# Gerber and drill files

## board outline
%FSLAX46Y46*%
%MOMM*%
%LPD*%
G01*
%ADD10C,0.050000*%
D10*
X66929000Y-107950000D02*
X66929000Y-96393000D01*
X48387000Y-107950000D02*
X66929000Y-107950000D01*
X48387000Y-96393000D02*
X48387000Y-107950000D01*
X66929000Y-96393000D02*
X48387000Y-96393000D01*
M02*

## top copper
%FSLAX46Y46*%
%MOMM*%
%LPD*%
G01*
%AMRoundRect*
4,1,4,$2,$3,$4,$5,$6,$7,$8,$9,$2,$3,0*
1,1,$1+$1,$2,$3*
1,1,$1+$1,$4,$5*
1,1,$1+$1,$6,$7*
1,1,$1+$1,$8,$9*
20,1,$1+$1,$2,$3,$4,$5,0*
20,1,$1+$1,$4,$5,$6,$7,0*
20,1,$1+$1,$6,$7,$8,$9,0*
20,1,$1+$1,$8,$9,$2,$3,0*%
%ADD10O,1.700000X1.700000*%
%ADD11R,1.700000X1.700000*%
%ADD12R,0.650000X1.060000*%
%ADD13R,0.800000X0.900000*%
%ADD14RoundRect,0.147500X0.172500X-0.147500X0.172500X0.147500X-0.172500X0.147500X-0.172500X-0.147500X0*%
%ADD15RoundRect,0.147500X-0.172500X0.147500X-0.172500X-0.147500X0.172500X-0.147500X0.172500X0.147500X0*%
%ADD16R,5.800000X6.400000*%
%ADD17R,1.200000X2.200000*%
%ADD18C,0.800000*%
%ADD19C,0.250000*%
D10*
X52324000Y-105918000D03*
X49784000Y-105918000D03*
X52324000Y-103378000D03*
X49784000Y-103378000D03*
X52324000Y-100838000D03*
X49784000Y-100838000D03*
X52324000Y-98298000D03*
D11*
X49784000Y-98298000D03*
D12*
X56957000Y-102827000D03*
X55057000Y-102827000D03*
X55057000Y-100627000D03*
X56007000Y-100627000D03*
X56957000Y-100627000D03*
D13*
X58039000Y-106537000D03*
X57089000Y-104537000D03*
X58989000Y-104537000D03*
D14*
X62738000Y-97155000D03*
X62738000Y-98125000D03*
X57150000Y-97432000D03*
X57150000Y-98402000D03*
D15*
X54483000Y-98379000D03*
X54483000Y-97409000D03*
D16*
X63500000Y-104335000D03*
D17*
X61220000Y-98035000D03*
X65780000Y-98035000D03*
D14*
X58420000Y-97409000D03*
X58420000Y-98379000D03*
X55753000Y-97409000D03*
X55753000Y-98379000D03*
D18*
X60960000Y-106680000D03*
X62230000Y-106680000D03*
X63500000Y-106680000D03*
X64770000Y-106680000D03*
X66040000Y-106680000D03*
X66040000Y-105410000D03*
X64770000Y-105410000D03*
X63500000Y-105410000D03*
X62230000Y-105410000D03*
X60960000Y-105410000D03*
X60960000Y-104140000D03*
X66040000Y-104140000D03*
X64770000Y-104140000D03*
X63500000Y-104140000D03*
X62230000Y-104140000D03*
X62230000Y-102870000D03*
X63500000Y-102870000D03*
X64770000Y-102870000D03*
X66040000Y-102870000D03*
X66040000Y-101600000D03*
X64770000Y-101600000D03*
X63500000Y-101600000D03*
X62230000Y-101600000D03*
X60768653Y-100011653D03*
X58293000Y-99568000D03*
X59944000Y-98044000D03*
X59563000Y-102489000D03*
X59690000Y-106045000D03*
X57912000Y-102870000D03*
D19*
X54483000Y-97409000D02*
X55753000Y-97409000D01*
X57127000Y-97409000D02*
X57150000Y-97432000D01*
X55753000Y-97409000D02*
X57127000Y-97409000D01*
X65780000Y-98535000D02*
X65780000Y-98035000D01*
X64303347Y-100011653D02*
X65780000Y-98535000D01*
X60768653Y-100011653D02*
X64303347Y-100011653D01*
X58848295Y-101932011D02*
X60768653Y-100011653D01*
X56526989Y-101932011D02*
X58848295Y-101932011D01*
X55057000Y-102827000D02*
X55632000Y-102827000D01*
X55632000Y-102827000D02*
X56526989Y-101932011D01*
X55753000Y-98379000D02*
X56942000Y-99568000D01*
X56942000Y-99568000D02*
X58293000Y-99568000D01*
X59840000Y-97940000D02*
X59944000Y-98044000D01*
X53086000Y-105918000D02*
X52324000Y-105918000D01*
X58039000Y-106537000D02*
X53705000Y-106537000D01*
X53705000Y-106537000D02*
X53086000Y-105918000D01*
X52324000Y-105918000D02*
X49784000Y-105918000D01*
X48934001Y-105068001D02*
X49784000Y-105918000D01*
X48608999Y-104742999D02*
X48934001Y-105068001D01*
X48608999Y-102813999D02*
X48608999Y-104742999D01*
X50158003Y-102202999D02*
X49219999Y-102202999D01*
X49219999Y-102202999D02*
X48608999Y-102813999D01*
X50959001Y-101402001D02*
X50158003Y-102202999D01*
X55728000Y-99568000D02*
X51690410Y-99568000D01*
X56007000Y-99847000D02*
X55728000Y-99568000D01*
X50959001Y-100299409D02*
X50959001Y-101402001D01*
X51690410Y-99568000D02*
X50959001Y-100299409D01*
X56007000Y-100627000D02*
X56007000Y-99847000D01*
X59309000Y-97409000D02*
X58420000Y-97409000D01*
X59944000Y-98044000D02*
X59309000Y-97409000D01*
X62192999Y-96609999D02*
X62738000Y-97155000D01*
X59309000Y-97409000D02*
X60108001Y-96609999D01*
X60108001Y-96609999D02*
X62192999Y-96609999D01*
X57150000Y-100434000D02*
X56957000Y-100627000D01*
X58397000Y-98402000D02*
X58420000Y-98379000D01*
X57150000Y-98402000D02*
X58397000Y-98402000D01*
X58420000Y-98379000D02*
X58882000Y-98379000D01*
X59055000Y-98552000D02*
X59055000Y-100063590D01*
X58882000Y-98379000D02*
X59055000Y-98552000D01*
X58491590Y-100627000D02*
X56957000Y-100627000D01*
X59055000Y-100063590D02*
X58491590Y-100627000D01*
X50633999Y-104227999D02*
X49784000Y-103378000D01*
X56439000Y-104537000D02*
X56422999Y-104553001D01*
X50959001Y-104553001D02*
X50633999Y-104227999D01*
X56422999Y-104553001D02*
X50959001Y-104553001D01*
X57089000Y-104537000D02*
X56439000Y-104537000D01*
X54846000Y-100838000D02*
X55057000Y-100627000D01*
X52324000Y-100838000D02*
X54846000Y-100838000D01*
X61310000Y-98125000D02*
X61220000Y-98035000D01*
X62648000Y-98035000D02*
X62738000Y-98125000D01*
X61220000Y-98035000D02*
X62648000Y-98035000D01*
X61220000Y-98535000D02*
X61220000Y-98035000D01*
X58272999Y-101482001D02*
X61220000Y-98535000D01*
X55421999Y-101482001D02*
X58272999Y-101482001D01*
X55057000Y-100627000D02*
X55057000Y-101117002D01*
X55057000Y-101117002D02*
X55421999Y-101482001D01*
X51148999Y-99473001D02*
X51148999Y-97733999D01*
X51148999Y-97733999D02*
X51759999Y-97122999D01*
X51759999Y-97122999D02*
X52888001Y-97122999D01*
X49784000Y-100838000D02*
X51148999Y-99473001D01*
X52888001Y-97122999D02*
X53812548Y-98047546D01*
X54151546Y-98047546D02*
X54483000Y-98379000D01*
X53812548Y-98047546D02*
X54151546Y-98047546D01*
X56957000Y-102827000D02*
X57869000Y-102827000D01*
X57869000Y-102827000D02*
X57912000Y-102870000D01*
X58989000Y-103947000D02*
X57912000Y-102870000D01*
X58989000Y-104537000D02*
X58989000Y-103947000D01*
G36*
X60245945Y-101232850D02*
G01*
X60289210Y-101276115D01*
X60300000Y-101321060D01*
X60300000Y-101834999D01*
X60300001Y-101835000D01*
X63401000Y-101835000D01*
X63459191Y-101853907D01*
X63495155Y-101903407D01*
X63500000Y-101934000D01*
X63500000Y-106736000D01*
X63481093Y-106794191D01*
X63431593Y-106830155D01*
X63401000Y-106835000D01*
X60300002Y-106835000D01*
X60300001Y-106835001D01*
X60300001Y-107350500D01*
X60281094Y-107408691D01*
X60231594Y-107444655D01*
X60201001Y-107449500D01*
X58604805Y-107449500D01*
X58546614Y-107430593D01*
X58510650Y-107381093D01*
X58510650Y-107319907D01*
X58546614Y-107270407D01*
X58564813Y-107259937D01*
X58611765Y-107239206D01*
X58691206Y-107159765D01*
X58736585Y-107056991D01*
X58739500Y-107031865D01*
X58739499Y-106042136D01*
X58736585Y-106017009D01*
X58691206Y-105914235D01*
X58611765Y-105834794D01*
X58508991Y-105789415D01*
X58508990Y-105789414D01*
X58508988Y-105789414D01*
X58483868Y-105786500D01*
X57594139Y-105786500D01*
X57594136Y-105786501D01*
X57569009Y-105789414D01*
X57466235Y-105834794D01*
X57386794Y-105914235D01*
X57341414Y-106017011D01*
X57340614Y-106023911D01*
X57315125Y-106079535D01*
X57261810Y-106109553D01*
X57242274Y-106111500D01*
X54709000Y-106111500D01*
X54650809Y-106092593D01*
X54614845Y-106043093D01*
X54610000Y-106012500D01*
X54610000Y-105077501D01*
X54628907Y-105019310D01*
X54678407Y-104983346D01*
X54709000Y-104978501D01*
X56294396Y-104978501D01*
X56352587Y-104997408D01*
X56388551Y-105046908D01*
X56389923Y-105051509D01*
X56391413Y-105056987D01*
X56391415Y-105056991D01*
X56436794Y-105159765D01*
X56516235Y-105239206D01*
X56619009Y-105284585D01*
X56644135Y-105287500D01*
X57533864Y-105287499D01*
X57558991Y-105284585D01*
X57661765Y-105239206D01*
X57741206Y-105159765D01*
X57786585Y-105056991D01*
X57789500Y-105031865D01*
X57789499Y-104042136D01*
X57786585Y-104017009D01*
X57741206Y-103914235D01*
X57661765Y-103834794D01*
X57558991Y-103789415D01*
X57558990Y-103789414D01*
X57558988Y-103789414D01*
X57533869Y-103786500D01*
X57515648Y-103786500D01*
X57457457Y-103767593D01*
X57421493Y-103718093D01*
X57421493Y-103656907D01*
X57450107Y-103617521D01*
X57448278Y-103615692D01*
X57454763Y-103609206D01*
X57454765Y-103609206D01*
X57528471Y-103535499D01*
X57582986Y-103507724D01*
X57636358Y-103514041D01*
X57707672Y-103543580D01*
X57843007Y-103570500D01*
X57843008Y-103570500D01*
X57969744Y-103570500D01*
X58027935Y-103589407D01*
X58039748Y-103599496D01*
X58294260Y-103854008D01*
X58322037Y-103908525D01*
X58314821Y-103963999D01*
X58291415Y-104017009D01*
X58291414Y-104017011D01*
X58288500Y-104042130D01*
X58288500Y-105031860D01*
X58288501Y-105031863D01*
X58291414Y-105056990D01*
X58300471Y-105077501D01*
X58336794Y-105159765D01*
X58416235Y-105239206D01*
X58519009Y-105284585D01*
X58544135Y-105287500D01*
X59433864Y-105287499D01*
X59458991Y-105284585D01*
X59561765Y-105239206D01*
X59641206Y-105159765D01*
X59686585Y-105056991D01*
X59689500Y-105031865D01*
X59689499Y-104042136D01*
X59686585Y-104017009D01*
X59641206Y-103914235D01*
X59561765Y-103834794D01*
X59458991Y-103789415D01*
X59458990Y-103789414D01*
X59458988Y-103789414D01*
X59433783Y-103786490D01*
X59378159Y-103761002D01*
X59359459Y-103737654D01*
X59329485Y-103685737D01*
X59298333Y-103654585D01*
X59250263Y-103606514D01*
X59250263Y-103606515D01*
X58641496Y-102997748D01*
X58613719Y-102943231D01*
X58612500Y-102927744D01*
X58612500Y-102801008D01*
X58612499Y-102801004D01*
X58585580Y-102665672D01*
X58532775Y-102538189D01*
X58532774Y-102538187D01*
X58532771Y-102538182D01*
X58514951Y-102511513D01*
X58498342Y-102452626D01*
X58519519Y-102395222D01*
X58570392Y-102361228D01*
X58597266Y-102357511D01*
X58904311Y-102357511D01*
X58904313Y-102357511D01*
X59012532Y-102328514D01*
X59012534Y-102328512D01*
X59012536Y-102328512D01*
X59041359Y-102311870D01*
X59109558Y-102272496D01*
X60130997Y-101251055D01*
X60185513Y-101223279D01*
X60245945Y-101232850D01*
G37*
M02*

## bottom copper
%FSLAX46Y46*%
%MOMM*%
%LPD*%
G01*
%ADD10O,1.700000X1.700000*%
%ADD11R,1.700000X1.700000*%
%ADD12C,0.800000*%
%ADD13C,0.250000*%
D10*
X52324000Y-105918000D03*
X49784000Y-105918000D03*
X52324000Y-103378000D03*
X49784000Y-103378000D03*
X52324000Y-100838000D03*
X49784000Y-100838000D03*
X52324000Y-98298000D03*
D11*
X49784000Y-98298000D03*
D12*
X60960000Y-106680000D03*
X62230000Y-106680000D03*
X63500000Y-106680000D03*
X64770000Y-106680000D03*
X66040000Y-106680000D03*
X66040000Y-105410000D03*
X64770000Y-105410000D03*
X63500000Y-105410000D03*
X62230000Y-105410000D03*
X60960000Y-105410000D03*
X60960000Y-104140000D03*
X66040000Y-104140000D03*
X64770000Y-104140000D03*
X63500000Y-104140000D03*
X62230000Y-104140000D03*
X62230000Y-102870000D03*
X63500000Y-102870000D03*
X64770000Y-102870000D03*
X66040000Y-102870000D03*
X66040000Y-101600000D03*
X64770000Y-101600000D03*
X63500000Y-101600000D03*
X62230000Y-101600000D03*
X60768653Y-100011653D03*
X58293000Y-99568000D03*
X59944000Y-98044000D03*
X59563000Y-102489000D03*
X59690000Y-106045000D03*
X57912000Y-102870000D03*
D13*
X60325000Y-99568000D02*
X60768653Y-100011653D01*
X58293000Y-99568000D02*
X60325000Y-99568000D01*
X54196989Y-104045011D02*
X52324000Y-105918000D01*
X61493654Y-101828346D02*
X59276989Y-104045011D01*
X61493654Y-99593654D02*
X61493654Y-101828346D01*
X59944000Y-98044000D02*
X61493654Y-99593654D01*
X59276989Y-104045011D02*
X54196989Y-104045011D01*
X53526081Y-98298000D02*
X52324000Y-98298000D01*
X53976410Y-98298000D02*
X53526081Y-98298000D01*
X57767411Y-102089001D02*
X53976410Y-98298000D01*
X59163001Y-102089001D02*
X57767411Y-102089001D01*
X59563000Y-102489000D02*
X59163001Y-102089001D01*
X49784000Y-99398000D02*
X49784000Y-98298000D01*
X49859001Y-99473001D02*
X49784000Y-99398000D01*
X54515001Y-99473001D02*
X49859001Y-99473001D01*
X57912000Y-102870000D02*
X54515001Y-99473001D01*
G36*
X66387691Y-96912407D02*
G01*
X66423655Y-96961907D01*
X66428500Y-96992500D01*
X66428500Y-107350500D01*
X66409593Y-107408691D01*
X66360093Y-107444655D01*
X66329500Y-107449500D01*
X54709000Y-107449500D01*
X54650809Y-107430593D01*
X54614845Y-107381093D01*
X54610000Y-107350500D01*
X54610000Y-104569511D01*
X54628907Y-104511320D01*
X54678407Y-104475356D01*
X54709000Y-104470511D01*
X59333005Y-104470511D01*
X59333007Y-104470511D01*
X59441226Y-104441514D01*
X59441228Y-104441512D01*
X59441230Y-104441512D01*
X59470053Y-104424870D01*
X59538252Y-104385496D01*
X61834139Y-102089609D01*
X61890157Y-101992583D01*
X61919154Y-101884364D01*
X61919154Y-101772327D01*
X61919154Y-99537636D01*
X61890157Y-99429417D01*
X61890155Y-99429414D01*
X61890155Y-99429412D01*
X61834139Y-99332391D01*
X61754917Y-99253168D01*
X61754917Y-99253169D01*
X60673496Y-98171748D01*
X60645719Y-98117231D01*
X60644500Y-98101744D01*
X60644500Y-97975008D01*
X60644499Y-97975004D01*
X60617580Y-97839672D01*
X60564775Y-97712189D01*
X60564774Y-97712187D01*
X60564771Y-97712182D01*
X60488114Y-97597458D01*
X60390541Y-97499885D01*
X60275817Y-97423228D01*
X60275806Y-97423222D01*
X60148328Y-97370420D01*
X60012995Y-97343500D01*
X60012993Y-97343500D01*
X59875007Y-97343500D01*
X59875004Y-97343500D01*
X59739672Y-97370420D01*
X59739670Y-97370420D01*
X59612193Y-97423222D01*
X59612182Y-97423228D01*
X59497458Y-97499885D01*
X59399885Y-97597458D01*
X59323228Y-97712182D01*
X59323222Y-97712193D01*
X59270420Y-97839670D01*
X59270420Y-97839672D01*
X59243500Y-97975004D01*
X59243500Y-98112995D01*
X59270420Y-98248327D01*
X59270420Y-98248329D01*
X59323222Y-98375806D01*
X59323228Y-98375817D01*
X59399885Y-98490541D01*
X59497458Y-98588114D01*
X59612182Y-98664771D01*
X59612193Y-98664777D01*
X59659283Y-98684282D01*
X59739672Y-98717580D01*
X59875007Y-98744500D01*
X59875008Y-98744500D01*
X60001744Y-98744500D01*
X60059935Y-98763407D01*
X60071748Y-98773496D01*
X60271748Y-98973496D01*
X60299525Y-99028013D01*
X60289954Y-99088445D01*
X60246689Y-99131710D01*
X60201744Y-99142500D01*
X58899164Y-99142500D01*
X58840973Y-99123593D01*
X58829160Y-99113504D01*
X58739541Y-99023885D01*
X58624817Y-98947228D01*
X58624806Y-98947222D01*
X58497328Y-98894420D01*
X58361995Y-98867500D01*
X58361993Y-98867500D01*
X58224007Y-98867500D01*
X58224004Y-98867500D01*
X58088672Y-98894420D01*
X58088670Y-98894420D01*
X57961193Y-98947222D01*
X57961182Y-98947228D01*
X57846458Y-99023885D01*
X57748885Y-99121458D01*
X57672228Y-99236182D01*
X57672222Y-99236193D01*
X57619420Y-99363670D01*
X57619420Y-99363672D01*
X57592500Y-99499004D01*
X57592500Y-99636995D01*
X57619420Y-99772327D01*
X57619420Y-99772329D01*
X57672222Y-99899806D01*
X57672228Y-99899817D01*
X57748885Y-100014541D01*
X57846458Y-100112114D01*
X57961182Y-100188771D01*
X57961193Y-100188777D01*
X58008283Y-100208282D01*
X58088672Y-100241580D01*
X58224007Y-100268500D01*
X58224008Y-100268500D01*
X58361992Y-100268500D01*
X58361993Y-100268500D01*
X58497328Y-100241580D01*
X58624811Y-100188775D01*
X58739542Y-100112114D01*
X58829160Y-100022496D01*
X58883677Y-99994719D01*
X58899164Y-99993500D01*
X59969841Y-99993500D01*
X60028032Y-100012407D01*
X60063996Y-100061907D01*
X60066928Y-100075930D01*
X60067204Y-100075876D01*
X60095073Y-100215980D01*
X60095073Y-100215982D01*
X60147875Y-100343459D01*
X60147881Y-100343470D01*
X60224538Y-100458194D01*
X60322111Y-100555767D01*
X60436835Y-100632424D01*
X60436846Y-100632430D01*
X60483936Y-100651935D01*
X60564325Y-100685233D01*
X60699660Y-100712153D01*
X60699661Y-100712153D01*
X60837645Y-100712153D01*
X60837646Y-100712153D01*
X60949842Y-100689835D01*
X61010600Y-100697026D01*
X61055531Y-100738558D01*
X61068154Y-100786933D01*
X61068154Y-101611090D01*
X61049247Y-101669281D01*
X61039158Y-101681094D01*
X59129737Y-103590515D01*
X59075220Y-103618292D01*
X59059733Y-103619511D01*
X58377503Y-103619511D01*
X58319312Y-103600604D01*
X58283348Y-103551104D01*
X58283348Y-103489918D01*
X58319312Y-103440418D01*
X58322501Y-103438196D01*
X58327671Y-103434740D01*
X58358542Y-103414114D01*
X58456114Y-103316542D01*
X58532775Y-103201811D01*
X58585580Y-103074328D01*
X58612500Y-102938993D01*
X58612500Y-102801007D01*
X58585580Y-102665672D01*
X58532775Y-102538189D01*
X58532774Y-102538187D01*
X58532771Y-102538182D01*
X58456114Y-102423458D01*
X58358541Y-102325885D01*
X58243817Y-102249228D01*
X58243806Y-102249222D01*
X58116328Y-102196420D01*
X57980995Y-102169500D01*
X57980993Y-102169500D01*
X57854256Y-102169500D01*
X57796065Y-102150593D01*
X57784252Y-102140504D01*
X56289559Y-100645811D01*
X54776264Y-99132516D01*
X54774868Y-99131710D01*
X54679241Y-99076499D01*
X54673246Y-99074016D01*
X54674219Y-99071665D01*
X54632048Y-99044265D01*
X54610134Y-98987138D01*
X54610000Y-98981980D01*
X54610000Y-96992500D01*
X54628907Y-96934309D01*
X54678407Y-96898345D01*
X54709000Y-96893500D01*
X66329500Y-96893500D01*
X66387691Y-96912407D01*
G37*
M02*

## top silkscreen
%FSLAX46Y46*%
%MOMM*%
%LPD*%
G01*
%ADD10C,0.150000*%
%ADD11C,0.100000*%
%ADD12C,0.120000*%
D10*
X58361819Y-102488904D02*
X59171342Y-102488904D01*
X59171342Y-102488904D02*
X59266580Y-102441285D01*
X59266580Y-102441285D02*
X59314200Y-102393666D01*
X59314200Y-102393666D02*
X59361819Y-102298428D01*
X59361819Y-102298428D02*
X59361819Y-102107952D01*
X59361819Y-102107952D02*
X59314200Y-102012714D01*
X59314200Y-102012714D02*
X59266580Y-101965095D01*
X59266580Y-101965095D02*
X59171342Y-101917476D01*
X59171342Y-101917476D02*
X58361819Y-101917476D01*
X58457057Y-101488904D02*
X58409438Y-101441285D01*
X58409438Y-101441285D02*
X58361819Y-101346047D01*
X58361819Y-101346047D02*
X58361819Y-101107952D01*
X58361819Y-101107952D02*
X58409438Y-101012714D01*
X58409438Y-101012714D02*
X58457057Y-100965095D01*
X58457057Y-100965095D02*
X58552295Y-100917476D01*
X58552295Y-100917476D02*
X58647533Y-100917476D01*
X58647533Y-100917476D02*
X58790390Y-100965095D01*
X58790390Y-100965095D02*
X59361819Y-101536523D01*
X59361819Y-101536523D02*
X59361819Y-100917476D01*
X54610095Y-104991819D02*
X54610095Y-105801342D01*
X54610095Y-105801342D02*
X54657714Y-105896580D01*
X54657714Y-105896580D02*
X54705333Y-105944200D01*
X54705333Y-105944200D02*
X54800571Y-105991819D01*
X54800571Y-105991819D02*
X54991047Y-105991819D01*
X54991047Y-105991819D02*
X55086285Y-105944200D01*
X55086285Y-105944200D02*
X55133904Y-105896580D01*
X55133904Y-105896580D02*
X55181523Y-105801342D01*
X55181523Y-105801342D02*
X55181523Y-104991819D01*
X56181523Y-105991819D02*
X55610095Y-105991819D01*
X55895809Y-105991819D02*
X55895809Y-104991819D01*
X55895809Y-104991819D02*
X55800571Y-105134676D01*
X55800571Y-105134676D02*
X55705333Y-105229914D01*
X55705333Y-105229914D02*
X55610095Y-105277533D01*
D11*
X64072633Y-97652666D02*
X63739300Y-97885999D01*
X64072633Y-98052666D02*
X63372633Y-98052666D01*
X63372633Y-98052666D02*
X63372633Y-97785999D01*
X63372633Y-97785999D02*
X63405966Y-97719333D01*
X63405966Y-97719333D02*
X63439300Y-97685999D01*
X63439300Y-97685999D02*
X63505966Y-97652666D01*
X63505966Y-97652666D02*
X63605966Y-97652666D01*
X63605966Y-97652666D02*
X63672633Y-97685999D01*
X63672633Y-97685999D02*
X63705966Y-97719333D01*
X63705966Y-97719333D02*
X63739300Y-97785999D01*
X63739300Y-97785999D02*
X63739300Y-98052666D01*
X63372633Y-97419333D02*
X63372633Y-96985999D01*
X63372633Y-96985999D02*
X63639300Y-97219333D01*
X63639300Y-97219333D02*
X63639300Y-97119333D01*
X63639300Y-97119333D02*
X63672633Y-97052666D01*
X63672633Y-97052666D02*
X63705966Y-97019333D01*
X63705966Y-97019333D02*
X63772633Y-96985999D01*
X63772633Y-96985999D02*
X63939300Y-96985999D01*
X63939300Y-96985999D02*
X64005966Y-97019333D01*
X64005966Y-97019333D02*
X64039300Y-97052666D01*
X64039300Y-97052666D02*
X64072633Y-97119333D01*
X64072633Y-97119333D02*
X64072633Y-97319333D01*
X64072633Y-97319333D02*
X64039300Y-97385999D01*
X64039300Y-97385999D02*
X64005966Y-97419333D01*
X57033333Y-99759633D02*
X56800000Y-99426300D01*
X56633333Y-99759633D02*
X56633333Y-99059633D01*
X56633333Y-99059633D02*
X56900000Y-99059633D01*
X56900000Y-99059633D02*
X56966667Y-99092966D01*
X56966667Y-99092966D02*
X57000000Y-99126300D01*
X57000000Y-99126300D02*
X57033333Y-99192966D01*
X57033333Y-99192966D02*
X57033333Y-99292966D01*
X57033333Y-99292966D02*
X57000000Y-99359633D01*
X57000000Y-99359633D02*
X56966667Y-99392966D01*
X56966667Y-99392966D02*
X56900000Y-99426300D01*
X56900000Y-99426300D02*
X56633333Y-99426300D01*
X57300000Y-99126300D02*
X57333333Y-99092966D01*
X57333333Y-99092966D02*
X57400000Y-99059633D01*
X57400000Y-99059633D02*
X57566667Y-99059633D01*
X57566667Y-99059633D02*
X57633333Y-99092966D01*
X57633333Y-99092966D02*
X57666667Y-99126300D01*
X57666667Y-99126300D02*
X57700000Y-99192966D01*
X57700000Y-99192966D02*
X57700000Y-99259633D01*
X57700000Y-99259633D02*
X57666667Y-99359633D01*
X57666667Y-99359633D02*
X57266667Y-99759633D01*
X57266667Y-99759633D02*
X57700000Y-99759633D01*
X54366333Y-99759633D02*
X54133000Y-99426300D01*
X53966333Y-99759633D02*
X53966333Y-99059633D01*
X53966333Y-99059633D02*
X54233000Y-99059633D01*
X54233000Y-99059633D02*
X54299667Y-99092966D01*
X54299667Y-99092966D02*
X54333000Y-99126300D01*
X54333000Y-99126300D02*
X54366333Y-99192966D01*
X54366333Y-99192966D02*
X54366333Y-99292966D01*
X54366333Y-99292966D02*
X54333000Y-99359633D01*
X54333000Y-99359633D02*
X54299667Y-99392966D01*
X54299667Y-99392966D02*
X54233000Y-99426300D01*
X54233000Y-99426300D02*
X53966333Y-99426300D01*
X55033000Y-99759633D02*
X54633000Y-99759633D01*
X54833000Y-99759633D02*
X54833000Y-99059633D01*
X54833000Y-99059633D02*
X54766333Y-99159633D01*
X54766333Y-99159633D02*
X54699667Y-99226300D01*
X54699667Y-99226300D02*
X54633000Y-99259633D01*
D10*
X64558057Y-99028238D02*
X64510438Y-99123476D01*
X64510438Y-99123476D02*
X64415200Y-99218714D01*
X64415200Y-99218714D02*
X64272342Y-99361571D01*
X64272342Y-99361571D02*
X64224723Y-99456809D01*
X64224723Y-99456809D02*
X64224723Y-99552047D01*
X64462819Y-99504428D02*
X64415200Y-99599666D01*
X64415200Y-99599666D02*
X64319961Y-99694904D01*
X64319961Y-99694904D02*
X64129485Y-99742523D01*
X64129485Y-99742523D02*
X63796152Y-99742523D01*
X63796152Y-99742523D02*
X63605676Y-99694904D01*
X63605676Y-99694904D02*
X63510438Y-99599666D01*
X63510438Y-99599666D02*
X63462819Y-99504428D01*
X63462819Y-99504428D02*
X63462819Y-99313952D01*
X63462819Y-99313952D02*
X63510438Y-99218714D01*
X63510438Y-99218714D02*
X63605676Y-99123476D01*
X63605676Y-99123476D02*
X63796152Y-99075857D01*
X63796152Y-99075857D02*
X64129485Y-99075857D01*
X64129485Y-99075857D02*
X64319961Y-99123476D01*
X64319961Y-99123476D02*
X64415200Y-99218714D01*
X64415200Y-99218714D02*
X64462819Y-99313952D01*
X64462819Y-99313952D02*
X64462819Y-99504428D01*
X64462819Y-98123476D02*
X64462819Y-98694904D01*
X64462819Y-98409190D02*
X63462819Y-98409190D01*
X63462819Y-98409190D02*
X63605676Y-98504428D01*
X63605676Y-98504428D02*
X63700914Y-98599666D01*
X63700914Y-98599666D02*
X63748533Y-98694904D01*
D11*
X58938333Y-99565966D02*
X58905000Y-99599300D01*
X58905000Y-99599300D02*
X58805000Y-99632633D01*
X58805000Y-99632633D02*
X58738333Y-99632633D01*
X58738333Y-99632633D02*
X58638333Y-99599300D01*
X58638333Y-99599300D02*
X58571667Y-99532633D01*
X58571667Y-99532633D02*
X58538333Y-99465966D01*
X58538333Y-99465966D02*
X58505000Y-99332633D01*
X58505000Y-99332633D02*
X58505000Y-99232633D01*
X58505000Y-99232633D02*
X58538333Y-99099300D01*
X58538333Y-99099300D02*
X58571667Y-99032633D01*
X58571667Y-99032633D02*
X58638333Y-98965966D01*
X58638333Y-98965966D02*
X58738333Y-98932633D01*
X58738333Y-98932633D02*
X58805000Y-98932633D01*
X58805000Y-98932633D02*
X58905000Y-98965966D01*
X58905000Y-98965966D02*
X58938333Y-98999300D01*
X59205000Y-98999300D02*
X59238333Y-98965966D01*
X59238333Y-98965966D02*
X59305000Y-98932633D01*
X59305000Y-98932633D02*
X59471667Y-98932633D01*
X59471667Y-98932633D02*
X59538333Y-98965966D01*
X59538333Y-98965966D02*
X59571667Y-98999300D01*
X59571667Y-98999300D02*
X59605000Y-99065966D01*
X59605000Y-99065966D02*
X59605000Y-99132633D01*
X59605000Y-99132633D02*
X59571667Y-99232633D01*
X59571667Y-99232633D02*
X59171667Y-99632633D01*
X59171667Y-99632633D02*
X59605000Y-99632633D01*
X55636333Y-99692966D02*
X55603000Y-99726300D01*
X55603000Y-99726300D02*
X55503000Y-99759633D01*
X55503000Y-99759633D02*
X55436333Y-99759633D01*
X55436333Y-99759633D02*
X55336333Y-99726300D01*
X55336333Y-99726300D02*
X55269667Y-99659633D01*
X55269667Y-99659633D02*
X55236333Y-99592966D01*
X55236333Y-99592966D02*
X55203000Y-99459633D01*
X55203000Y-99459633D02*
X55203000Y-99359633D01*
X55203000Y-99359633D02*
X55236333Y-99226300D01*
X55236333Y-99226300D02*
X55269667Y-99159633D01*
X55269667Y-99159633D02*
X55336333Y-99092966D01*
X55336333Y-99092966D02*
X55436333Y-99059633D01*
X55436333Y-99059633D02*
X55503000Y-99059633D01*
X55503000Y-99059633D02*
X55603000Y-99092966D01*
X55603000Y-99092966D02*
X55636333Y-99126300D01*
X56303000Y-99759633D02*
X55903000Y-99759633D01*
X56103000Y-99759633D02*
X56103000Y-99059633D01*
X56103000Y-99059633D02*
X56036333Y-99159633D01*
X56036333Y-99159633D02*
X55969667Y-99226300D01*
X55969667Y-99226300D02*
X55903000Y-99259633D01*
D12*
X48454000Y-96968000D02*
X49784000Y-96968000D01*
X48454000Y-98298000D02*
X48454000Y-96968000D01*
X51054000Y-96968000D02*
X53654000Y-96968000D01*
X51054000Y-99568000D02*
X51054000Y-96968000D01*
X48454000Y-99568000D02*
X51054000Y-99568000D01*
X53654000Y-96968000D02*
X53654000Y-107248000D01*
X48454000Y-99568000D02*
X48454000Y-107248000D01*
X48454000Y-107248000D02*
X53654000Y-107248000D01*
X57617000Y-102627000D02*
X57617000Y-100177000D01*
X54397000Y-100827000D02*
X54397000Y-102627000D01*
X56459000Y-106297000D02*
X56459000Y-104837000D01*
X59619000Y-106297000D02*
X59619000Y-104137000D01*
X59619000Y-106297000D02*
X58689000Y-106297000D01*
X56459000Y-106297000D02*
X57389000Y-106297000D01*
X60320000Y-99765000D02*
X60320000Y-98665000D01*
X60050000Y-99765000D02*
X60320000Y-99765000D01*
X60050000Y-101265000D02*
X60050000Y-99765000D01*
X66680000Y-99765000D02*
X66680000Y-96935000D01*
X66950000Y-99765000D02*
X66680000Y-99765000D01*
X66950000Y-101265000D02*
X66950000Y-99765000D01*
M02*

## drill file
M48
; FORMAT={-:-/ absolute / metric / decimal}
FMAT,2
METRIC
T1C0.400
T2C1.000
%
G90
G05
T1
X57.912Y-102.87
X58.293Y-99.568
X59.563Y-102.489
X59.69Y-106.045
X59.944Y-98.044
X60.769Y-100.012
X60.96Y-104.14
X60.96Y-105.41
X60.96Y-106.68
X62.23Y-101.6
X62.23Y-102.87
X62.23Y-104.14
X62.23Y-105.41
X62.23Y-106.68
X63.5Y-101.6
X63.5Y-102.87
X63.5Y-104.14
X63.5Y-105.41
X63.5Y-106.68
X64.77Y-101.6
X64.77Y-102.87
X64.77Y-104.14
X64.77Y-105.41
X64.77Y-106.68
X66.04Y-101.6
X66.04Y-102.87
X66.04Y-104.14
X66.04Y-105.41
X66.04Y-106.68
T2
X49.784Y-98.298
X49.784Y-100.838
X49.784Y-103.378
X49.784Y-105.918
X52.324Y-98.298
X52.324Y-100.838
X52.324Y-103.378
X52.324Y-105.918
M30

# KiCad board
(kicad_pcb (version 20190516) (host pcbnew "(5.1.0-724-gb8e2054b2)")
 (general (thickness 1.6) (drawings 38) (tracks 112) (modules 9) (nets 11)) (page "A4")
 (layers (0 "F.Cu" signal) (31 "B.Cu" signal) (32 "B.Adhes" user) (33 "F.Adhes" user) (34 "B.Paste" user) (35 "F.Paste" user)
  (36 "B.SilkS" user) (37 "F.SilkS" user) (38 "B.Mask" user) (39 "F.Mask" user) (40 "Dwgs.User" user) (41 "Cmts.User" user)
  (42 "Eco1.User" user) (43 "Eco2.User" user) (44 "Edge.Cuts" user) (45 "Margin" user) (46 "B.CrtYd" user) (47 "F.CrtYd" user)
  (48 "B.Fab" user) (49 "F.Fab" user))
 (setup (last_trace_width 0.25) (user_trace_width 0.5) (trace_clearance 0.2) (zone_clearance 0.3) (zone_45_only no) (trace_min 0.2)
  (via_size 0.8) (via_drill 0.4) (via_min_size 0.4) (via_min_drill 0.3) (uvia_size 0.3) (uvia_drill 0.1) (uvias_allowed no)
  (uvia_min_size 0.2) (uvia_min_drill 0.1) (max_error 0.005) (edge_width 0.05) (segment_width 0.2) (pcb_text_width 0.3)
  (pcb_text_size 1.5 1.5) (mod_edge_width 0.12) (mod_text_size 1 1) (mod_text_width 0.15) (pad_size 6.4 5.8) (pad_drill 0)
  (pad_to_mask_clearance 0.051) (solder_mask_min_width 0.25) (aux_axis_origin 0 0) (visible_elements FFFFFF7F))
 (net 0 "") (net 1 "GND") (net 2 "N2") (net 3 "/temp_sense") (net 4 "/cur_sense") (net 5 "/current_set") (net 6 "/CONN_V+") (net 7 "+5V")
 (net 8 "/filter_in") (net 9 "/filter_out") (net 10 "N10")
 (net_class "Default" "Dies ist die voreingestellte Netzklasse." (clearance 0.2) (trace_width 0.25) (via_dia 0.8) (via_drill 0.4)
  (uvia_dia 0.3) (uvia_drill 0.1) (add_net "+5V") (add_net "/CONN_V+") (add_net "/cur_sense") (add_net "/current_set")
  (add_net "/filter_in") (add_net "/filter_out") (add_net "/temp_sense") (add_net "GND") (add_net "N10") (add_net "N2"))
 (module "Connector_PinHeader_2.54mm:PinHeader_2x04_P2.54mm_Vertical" (layer "F.Cu") (at 49.784 98.298)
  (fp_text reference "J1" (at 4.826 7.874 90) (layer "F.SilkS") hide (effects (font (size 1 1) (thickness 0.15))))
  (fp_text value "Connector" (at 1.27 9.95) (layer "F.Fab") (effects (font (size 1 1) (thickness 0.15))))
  (fp_line (start -1.33 -1.33) (end 0 -1.33) (layer "F.SilkS") (width 0.12))
  (fp_line (start -1.33 0) (end -1.33 -1.33) (layer "F.SilkS") (width 0.12))
  (fp_line (start 1.27 -1.33) (end 3.87 -1.33) (layer "F.SilkS") (width 0.12))
  (fp_line (start 1.27 1.27) (end 1.27 -1.33) (layer "F.SilkS") (width 0.12))
  (fp_line (start -1.33 1.27) (end 1.27 1.27) (layer "F.SilkS") (width 0.12))
  (fp_line (start 3.87 -1.33) (end 3.87 8.95) (layer "F.SilkS") (width 0.12))
  (fp_line (start -1.33 1.27) (end -1.33 8.95) (layer "F.SilkS") (width 0.12))
  (fp_line (start -1.33 8.95) (end 3.87 8.95) (layer "F.SilkS") (width 0.12))
  (pad "8" thru_hole oval (at 2.54 7.62) (size 1.7 1.7) (drill 1) (layers *.Cu *.Mask) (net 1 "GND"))
  (pad "7" thru_hole oval (at 0 7.62) (size 1.7 1.7) (drill 1) (layers *.Cu *.Mask) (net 1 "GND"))
  (pad "6" thru_hole oval (at 2.54 5.08) (size 1.7 1.7) (drill 1) (layers *.Cu *.Mask) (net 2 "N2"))
  (pad "5" thru_hole oval (at 0 5.08) (size 1.7 1.7) (drill 1) (layers *.Cu *.Mask) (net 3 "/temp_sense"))
  (pad "4" thru_hole oval (at 2.54 2.54) (size 1.7 1.7) (drill 1) (layers *.Cu *.Mask) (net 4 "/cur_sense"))
  (pad "3" thru_hole oval (at 0 2.54) (size 1.7 1.7) (drill 1) (layers *.Cu *.Mask) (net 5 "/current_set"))
  (pad "2" thru_hole oval (at 2.54 0) (size 1.7 1.7) (drill 1) (layers *.Cu *.Mask) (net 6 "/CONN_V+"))
  (pad "1" thru_hole rect (at 0 0) (size 1.7 1.7) (drill 1) (layers *.Cu *.Mask) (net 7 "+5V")))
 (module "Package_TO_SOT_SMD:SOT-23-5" (layer "F.Cu") (at 56.007 101.727 270)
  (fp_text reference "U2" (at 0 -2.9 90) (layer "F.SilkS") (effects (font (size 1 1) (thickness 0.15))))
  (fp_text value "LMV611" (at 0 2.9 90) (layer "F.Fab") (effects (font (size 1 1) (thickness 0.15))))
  (fp_line (start 0.9 -1.61) (end -1.55 -1.61) (layer "F.SilkS") (width 0.12))
  (fp_line (start -0.9 1.61) (end 0.9 1.61) (layer "F.SilkS") (width 0.12))
  (pad "5" smd rect (at 1.1 -0.95 270) (size 1.06 0.65) (layers "F.Cu" "F.Paste" "F.Mask") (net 7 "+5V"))
  (pad "4" smd rect (at 1.1 0.95 270) (size 1.06 0.65) (layers "F.Cu" "F.Paste" "F.Mask") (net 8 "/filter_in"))
  (pad "3" smd rect (at -1.1 0.95 270) (size 1.06 0.65) (layers "F.Cu" "F.Paste" "F.Mask") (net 4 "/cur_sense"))
  (pad "2" smd rect (at -1.1 0 270) (size 1.06 0.65) (layers "F.Cu" "F.Paste" "F.Mask") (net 1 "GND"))
  (pad "1" smd rect (at -1.1 -0.95 270) (size 1.06 0.65) (layers "F.Cu" "F.Paste" "F.Mask") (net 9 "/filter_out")))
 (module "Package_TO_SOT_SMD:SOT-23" (layer "F.Cu") (at 58.039 105.537 270)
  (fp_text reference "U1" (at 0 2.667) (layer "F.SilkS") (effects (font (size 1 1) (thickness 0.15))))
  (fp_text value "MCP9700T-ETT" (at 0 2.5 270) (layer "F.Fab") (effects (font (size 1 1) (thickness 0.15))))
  (fp_line (start 0.76 1.58) (end -0.7 1.58) (layer "F.SilkS") (width 0.12))
  (fp_line (start 0.76 -1.58) (end -1.4 -1.58) (layer "F.SilkS") (width 0.12))
  (fp_line (start 0.76 -1.58) (end 0.76 -0.65) (layer "F.SilkS") (width 0.12))
  (fp_line (start 0.76 1.58) (end 0.76 0.65) (layer "F.SilkS") (width 0.12))
  (pad "3" smd rect (at 1 0 270) (size 0.9 0.8) (layers "F.Cu" "F.Paste" "F.Mask") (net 1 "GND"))
  (pad "2" smd rect (at -1 0.95 270) (size 0.9 0.8) (layers "F.Cu" "F.Paste" "F.Mask") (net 3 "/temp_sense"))
  (pad "1" smd rect (at -1 -0.95 270) (size 0.9 0.8) (layers "F.Cu" "F.Paste" "F.Mask") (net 7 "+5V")))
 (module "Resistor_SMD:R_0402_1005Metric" (layer "F.Cu") (at 62.738 97.64 90)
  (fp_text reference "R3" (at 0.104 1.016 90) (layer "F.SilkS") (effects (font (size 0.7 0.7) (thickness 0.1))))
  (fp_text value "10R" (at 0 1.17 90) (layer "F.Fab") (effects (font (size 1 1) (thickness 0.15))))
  (pad "2" smd roundrect (at 0.485 0 90) (size 0.59 0.64) (layers "F.Cu" "F.Paste" "F.Mask") (roundrect_rratio 0.25) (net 1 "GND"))
  (pad "1" smd roundrect (at -0.485 0 90) (size 0.59 0.64) (layers "F.Cu" "F.Paste" "F.Mask") (roundrect_rratio 0.25) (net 4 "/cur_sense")))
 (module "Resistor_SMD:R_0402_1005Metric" (layer "F.Cu") (at 57.15 97.917 90)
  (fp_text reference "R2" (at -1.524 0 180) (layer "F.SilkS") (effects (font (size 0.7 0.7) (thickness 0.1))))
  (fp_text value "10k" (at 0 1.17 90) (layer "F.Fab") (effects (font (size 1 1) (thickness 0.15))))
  (pad "2" smd roundrect (at 0.485 0 90) (size 0.59 0.64) (layers "F.Cu" "F.Paste" "F.Mask") (roundrect_rratio 0.25) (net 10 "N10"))
  (pad "1" smd roundrect (at -0.485 0 90) (size 0.59 0.64) (layers "F.Cu" "F.Paste" "F.Mask") (roundrect_rratio 0.25) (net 9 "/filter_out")))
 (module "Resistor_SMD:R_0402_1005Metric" (layer "F.Cu") (at 54.483 97.894 270)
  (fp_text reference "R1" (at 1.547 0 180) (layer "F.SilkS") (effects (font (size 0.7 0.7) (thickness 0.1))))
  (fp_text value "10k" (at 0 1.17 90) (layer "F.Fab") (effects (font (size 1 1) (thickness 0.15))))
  (pad "2" smd roundrect (at 0.485 0 270) (size 0.59 0.64) (layers "F.Cu" "F.Paste" "F.Mask") (roundrect_rratio 0.25) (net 5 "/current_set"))
  (pad "1" smd roundrect (at -0.485 0 270) (size 0.59 0.64) (layers "F.Cu" "F.Paste" "F.Mask") (roundrect_rratio 0.25) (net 10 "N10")))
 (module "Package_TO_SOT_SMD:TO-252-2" (layer "F.Cu") (at 63.5 102.235 270)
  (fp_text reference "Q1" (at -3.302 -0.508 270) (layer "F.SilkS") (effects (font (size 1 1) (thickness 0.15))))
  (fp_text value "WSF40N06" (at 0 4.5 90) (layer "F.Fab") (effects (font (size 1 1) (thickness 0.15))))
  (fp_line (start -2.47 3.18) (end -3.57 3.18) (layer "F.SilkS") (width 0.12))
  (fp_line (start -2.47 3.45) (end -2.47 3.18) (layer "F.SilkS") (width 0.12))
  (fp_line (start -0.97 3.45) (end -2.47 3.45) (layer "F.SilkS") (width 0.12))
  (fp_line (start -2.47 -3.18) (end -5.3 -3.18) (layer "F.SilkS") (width 0.12))
  (fp_line (start -2.47 -3.45) (end -2.47 -3.18) (layer "F.SilkS") (width 0.12))
  (fp_line (start -0.97 -3.45) (end -2.47 -3.45) (layer "F.SilkS") (width 0.12))
  (pad "" smd rect (at 0.425 1.525 270) (size 3.05 2.75) (layers "F.Paste"))
  (pad "" smd rect (at 3.775 -1.525 270) (size 3.05 2.75) (layers "F.Paste"))
  (pad "" smd rect (at 0.425 -1.525 270) (size 3.05 2.75) (layers "F.Paste"))
  (pad "" smd rect (at 3.775 1.525 270) (size 3.05 2.75) (layers "F.Paste"))
  (pad "2" smd rect (at 2.1 0 270) (size 6.4 5.8) (layers "F.Cu" "F.Mask") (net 6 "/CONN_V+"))
  (pad "3" smd rect (at -4.2 2.28 270) (size 2.2 1.2) (layers "F.Cu" "F.Paste" "F.Mask") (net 4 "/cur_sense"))
  (pad "1" smd rect (at -4.2 -2.28 270) (size 2.2 1.2) (layers "F.Cu" "F.Paste" "F.Mask") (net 8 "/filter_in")))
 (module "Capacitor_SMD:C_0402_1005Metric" (layer "F.Cu") (at 58.42 97.894 90)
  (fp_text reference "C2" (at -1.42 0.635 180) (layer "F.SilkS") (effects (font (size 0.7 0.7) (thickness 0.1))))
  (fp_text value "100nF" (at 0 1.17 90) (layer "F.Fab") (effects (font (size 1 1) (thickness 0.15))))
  (pad "2" smd roundrect (at 0.485 0 90) (size 0.59 0.64) (layers "F.Cu" "F.Paste" "F.Mask") (roundrect_rratio 0.25) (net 1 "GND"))
  (pad "1" smd roundrect (at -0.485 0 90) (size 0.59 0.64) (layers "F.Cu" "F.Paste" "F.Mask") (roundrect_rratio 0.25) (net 9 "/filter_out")))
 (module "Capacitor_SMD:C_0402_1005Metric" (layer "F.Cu") (at 55.753 97.894 90)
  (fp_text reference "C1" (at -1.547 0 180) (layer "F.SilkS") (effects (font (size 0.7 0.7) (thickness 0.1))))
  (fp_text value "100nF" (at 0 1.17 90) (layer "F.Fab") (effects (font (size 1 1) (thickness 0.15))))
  (pad "2" smd roundrect (at 0.485 0 90) (size 0.59 0.64) (layers "F.Cu" "F.Paste" "F.Mask") (roundrect_rratio 0.25) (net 10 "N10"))
  (pad "1" smd roundrect (at -0.485 0 90) (size 0.59 0.64) (layers "F.Cu" "F.Paste" "F.Mask") (roundrect_rratio 0.25) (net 8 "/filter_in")))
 (gr_line (start 66.929 107.95) (end 66.929 96.393) (layer "Edge.Cuts") (width 0.05))
 (gr_line (start 48.387 107.95) (end 66.929 107.95) (layer "Edge.Cuts") (width 0.05))
 (gr_line (start 48.387 96.393) (end 48.387 107.95) (layer "Edge.Cuts") (width 0.05))
 (gr_line (start 66.929 96.393) (end 48.387 96.393) (layer "Edge.Cuts") (width 0.05))
 (via (at 60.96 106.68) (size 0.8) (drill 0.4) (layers "F.Cu" "B.Cu") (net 6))
 (via (at 62.23 106.68) (size 0.8) (drill 0.4) (layers "F.Cu" "B.Cu") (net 6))
 (via (at 63.5 106.68) (size 0.8) (drill 0.4) (layers "F.Cu" "B.Cu") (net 6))
 (via (at 64.77 106.68) (size 0.8) (drill 0.4) (layers "F.Cu" "B.Cu") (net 6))
 (via (at 66.04 106.68) (size 0.8) (drill 0.4) (layers "F.Cu" "B.Cu") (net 6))
 (via (at 66.04 105.41) (size 0.8) (drill 0.4) (layers "F.Cu" "B.Cu") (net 6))
 (via (at 64.77 105.41) (size 0.8) (drill 0.4) (layers "F.Cu" "B.Cu") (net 6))
 (via (at 63.5 105.41) (size 0.8) (drill 0.4) (layers "F.Cu" "B.Cu") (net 6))
 (via (at 62.23 105.41) (size 0.8) (drill 0.4) (layers "F.Cu" "B.Cu") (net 6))
 (via (at 60.96 105.41) (size 0.8) (drill 0.4) (layers "F.Cu" "B.Cu") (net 6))
 (via (at 60.96 104.14) (size 0.8) (drill 0.4) (layers "F.Cu" "B.Cu") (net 6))
 (via (at 66.04 104.14) (size 0.8) (drill 0.4) (layers "F.Cu" "B.Cu") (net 6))
 (via (at 64.77 104.14) (size 0.8) (drill 0.4) (layers "F.Cu" "B.Cu") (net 6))
 (via (at 63.5 104.14) (size 0.8) (drill 0.4) (layers "F.Cu" "B.Cu") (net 6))
 (via (at 62.23 104.14) (size 0.8) (drill 0.4) (layers "F.Cu" "B.Cu") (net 6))
 (via (at 62.23 102.87) (size 0.8) (drill 0.4) (layers "F.Cu" "B.Cu") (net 6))
 (via (at 63.5 102.87) (size 0.8) (drill 0.4) (layers "F.Cu" "B.Cu") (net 6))
 (via (at 64.77 102.87) (size 0.8) (drill 0.4) (layers "F.Cu" "B.Cu") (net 6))
 (via (at 66.04 102.87) (size 0.8) (drill 0.4) (layers "F.Cu" "B.Cu") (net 6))
 (via (at 66.04 101.6) (size 0.8) (drill 0.4) (layers "F.Cu" "B.Cu") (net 6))
 (via (at 64.77 101.6) (size 0.8) (drill 0.4) (layers "F.Cu" "B.Cu") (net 6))
 (via (at 63.5 101.6) (size 0.8) (drill 0.4) (layers "F.Cu" "B.Cu") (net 6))
 (via (at 62.23 101.6) (size 0.8) (drill 0.4) (layers "F.Cu" "B.Cu") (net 6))
 (segment (start 54.483 97.409) (end 55.753 97.409) (width 0.25) (layer "F.Cu") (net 10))
 (segment (start 57.127 97.409) (end 57.15 97.432) (width 0.25) (layer "F.Cu") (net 10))
 (segment (start 55.753 97.409) (end 57.127 97.409) (width 0.25) (layer "F.Cu") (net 10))
 (via (at 60.768653 100.011653) (size 0.8) (drill 0.4) (layers "F.Cu" "B.Cu") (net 8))
 (segment (start 65.78 98.535) (end 65.78 98.035) (width 0.25) (layer "F.Cu") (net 8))
 (segment (start 64.303347 100.011653) (end 65.78 98.535) (width 0.25) (layer "F.Cu") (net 8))
 (segment (start 60.768653 100.011653) (end 64.303347 100.011653) (width 0.25) (layer "F.Cu") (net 8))
 (segment (start 58.848295 101.932011) (end 60.768653 100.011653) (width 0.25) (layer "F.Cu") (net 8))
 (segment (start 56.526989 101.932011) (end 58.848295 101.932011) (width 0.25) (layer "F.Cu") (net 8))
 (segment (start 55.057 102.827) (end 55.632 102.827) (width 0.25) (layer "F.Cu") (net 8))
 (segment (start 55.632 102.827) (end 56.526989 101.932011) (width 0.25) (layer "F.Cu") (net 8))
 (via (at 58.293 99.568) (size 0.8) (drill 0.4) (layers "F.Cu" "B.Cu") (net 8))
 (segment (start 55.753 98.379) (end 56.942 99.568) (width 0.25) (layer "F.Cu") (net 8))
 (segment (start 56.942 99.568) (end 58.293 99.568) (width 0.25) (layer "F.Cu") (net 8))
 (segment (start 60.325 99.568) (end 60.768653 100.011653) (width 0.25) (layer "B.Cu") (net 8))
 (segment (start 58.293 99.568) (end 60.325 99.568) (width 0.25) (layer "B.Cu") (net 8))
 (via (at 59.944 98.044) (size 0.8) (drill 0.4) (layers "F.Cu" "B.Cu") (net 1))
 (segment (start 59.84 97.94) (end 59.944 98.044) (width 0.25) (layer "F.Cu") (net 1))
 (segment (start 54.196989 104.045011) (end 52.324 105.918) (width 0.25) (layer "B.Cu") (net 1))
 (segment (start 53.086 105.918) (end 52.324 105.918) (width 0.25) (layer "F.Cu") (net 1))
 (segment (start 58.039 106.537) (end 53.705 106.537) (width 0.25) (layer "F.Cu") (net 1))
 (segment (start 53.705 106.537) (end 53.086 105.918) (width 0.25) (layer "F.Cu") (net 1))
 (segment (start 52.324 105.918) (end 49.784 105.918) (width 0.25) (layer "F.Cu") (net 1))
 (segment (start 48.934001 105.068001) (end 49.784 105.918) (width 0.25) (layer "F.Cu") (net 1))
 (segment (start 48.608999 104.742999) (end 48.934001 105.068001) (width 0.25) (layer "F.Cu") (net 1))
 (segment (start 48.608999 102.813999) (end 48.608999 104.742999) (width 0.25) (layer "F.Cu") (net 1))
 (segment (start 50.158003 102.202999) (end 49.219999 102.202999) (width 0.25) (layer "F.Cu") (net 1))
 (segment (start 49.219999 102.202999) (end 48.608999 102.813999) (width 0.25) (layer "F.Cu") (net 1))
 (segment (start 50.959001 101.402001) (end 50.158003 102.202999) (width 0.25) (layer "F.Cu") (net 1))
 (segment (start 55.728 99.568) (end 51.69041 99.568) (width 0.25) (layer "F.Cu") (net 1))
 (segment (start 56.007 99.847) (end 55.728 99.568) (width 0.25) (layer "F.Cu") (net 1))
 (segment (start 50.959001 100.299409) (end 50.959001 101.402001) (width 0.25) (layer "F.Cu") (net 1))
 (segment (start 51.69041 99.568) (end 50.959001 100.299409) (width 0.25) (layer "F.Cu") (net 1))
 (segment (start 56.007 100.627) (end 56.007 99.847) (width 0.25) (layer "F.Cu") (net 1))
 (segment (start 59.309 97.409) (end 58.42 97.409) (width 0.25) (layer "F.Cu") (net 1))
 (segment (start 59.944 98.044) (end 59.309 97.409) (width 0.25) (layer "F.Cu") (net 1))
 (segment (start 62.192999 96.609999) (end 62.738 97.155) (width 0.25) (layer "F.Cu") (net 1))
 (segment (start 59.309 97.409) (end 60.108001 96.609999) (width 0.25) (layer "F.Cu") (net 1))
 (segment (start 60.108001 96.609999) (end 62.192999 96.609999) (width 0.25) (layer "F.Cu") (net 1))
 (segment (start 61.493654 101.828346) (end 59.276989 104.045011) (width 0.25) (layer "B.Cu") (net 1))
 (segment (start 61.493654 99.593654) (end 61.493654 101.828346) (width 0.25) (layer "B.Cu") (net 1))
 (segment (start 59.944 98.044) (end 61.493654 99.593654) (width 0.25) (layer "B.Cu") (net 1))
 (segment (start 59.276989 104.045011) (end 54.196989 104.045011) (width 0.25) (layer "B.Cu") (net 1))
 (segment (start 57.15 100.434) (end 56.957 100.627) (width 0.25) (layer "F.Cu") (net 9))
 (segment (start 58.397 98.402) (end 58.42 98.379) (width 0.25) (layer "F.Cu") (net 9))
 (segment (start 57.15 98.402) (end 58.397 98.402) (width 0.25) (layer "F.Cu") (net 9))
 (segment (start 58.42 98.379) (end 58.882 98.379) (width 0.25) (layer "F.Cu") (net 9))
 (segment (start 59.055 98.552) (end 59.055 100.06359) (width 0.25) (layer "F.Cu") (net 9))
 (segment (start 58.882 98.379) (end 59.055 98.552) (width 0.25) (layer "F.Cu") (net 9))
 (segment (start 58.49159 100.627) (end 56.957 100.627) (width 0.25) (layer "F.Cu") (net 9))
 (segment (start 59.055 100.06359) (end 58.49159 100.627) (width 0.25) (layer "F.Cu") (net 9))
 (segment (start 50.633999 104.227999) (end 49.784 103.378) (width 0.25) (layer "F.Cu") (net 3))
 (segment (start 56.439 104.537) (end 56.422999 104.553001) (width 0.25) (layer "F.Cu") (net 3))
 (segment (start 50.959001 104.553001) (end 50.633999 104.227999) (width 0.25) (layer "F.Cu") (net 3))
 (segment (start 56.422999 104.553001) (end 50.959001 104.553001) (width 0.25) (layer "F.Cu") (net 3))
 (segment (start 57.089 104.537) (end 56.439 104.537) (width 0.25) (layer "F.Cu") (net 3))
 (segment (start 54.846 100.838) (end 55.057 100.627) (width 0.25) (layer "F.Cu") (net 4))
 (segment (start 52.324 100.838) (end 54.846 100.838) (width 0.25) (layer "F.Cu") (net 4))
 (segment (start 61.31 98.125) (end 61.22 98.035) (width 0.25) (layer "F.Cu") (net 4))
 (segment (start 62.648 98.035) (end 62.738 98.125) (width 0.25) (layer "F.Cu") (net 4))
 (segment (start 61.22 98.035) (end 62.648 98.035) (width 0.25) (layer "F.Cu") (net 4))
 (segment (start 61.22 98.535) (end 61.22 98.035) (width 0.25) (layer "F.Cu") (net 4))
 (segment (start 58.272999 101.482001) (end 61.22 98.535) (width 0.25) (layer "F.Cu") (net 4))
 (segment (start 55.421999 101.482001) (end 58.272999 101.482001) (width 0.25) (layer "F.Cu") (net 4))
 (segment (start 55.057 100.627) (end 55.057 101.117002) (width 0.25) (layer "F.Cu") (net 4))
 (segment (start 55.057 101.117002) (end 55.421999 101.482001) (width 0.25) (layer "F.Cu") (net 4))
 (segment (start 51.148999 99.473001) (end 51.148999 97.733999) (width 0.25) (layer "F.Cu") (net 5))
 (segment (start 51.148999 97.733999) (end 51.759999 97.122999) (width 0.25) (layer "F.Cu") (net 5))
 (segment (start 51.759999 97.122999) (end 52.888001 97.122999) (width 0.25) (layer "F.Cu") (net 5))
 (segment (start 49.784 100.838) (end 51.148999 99.473001) (width 0.25) (layer "F.Cu") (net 5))
 (segment (start 52.888001 97.122999) (end 53.812548 98.047546) (width 0.25) (layer "F.Cu") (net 5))
 (segment (start 54.151546 98.047546) (end 54.483 98.379) (width 0.25) (layer "F.Cu") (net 5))
 (segment (start 53.812548 98.047546) (end 54.151546 98.047546) (width 0.25) (layer "F.Cu") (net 5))
 (via (at 59.563 102.489) (size 0.8) (drill 0.4) (layers "F.Cu" "B.Cu") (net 6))
 (segment (start 53.526081 98.298) (end 52.324 98.298) (width 0.25) (layer "B.Cu") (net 6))
 (segment (start 53.97641 98.298) (end 53.526081 98.298) (width 0.25) (layer "B.Cu") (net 6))
 (segment (start 57.767411 102.089001) (end 53.97641 98.298) (width 0.25) (layer "B.Cu") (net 6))
 (segment (start 59.163001 102.089001) (end 57.767411 102.089001) (width 0.25) (layer "B.Cu") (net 6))
 (segment (start 59.563 102.489) (end 59.163001 102.089001) (width 0.25) (layer "B.Cu") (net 6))
 (via (at 59.69 106.045) (size 0.8) (drill 0.4) (layers "F.Cu" "B.Cu") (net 6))
 (via (at 57.912 102.87) (size 0.8) (drill 0.4) (layers "F.Cu" "B.Cu") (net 7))
 (segment (start 56.957 102.827) (end 57.869 102.827) (width 0.25) (layer "F.Cu") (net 7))
 (segment (start 57.869 102.827) (end 57.912 102.87) (width 0.25) (layer "F.Cu") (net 7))
 (segment (start 49.784 99.398) (end 49.784 98.298) (width 0.25) (layer "B.Cu") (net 7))
 (segment (start 49.859001 99.473001) (end 49.784 99.398) (width 0.25) (layer "B.Cu") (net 7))
 (segment (start 54.515001 99.473001) (end 49.859001 99.473001) (width 0.25) (layer "B.Cu") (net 7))
 (segment (start 57.912 102.87) (end 54.515001 99.473001) (width 0.25) (layer "B.Cu") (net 7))
 (segment (start 58.989 103.947) (end 57.912 102.87) (width 0.25) (layer "F.Cu") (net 7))
 (segment (start 58.989 104.537) (end 58.989 103.947) (width 0.25) (layer "F.Cu") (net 7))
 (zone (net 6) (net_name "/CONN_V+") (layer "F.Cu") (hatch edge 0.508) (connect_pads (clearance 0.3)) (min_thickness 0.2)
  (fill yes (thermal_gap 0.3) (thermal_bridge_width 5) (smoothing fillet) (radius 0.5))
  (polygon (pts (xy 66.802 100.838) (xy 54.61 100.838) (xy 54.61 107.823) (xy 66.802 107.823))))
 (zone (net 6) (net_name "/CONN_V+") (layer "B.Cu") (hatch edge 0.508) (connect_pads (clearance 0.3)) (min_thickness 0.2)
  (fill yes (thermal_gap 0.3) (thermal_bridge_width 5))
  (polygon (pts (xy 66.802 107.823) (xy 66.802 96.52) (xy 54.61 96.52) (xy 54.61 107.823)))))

